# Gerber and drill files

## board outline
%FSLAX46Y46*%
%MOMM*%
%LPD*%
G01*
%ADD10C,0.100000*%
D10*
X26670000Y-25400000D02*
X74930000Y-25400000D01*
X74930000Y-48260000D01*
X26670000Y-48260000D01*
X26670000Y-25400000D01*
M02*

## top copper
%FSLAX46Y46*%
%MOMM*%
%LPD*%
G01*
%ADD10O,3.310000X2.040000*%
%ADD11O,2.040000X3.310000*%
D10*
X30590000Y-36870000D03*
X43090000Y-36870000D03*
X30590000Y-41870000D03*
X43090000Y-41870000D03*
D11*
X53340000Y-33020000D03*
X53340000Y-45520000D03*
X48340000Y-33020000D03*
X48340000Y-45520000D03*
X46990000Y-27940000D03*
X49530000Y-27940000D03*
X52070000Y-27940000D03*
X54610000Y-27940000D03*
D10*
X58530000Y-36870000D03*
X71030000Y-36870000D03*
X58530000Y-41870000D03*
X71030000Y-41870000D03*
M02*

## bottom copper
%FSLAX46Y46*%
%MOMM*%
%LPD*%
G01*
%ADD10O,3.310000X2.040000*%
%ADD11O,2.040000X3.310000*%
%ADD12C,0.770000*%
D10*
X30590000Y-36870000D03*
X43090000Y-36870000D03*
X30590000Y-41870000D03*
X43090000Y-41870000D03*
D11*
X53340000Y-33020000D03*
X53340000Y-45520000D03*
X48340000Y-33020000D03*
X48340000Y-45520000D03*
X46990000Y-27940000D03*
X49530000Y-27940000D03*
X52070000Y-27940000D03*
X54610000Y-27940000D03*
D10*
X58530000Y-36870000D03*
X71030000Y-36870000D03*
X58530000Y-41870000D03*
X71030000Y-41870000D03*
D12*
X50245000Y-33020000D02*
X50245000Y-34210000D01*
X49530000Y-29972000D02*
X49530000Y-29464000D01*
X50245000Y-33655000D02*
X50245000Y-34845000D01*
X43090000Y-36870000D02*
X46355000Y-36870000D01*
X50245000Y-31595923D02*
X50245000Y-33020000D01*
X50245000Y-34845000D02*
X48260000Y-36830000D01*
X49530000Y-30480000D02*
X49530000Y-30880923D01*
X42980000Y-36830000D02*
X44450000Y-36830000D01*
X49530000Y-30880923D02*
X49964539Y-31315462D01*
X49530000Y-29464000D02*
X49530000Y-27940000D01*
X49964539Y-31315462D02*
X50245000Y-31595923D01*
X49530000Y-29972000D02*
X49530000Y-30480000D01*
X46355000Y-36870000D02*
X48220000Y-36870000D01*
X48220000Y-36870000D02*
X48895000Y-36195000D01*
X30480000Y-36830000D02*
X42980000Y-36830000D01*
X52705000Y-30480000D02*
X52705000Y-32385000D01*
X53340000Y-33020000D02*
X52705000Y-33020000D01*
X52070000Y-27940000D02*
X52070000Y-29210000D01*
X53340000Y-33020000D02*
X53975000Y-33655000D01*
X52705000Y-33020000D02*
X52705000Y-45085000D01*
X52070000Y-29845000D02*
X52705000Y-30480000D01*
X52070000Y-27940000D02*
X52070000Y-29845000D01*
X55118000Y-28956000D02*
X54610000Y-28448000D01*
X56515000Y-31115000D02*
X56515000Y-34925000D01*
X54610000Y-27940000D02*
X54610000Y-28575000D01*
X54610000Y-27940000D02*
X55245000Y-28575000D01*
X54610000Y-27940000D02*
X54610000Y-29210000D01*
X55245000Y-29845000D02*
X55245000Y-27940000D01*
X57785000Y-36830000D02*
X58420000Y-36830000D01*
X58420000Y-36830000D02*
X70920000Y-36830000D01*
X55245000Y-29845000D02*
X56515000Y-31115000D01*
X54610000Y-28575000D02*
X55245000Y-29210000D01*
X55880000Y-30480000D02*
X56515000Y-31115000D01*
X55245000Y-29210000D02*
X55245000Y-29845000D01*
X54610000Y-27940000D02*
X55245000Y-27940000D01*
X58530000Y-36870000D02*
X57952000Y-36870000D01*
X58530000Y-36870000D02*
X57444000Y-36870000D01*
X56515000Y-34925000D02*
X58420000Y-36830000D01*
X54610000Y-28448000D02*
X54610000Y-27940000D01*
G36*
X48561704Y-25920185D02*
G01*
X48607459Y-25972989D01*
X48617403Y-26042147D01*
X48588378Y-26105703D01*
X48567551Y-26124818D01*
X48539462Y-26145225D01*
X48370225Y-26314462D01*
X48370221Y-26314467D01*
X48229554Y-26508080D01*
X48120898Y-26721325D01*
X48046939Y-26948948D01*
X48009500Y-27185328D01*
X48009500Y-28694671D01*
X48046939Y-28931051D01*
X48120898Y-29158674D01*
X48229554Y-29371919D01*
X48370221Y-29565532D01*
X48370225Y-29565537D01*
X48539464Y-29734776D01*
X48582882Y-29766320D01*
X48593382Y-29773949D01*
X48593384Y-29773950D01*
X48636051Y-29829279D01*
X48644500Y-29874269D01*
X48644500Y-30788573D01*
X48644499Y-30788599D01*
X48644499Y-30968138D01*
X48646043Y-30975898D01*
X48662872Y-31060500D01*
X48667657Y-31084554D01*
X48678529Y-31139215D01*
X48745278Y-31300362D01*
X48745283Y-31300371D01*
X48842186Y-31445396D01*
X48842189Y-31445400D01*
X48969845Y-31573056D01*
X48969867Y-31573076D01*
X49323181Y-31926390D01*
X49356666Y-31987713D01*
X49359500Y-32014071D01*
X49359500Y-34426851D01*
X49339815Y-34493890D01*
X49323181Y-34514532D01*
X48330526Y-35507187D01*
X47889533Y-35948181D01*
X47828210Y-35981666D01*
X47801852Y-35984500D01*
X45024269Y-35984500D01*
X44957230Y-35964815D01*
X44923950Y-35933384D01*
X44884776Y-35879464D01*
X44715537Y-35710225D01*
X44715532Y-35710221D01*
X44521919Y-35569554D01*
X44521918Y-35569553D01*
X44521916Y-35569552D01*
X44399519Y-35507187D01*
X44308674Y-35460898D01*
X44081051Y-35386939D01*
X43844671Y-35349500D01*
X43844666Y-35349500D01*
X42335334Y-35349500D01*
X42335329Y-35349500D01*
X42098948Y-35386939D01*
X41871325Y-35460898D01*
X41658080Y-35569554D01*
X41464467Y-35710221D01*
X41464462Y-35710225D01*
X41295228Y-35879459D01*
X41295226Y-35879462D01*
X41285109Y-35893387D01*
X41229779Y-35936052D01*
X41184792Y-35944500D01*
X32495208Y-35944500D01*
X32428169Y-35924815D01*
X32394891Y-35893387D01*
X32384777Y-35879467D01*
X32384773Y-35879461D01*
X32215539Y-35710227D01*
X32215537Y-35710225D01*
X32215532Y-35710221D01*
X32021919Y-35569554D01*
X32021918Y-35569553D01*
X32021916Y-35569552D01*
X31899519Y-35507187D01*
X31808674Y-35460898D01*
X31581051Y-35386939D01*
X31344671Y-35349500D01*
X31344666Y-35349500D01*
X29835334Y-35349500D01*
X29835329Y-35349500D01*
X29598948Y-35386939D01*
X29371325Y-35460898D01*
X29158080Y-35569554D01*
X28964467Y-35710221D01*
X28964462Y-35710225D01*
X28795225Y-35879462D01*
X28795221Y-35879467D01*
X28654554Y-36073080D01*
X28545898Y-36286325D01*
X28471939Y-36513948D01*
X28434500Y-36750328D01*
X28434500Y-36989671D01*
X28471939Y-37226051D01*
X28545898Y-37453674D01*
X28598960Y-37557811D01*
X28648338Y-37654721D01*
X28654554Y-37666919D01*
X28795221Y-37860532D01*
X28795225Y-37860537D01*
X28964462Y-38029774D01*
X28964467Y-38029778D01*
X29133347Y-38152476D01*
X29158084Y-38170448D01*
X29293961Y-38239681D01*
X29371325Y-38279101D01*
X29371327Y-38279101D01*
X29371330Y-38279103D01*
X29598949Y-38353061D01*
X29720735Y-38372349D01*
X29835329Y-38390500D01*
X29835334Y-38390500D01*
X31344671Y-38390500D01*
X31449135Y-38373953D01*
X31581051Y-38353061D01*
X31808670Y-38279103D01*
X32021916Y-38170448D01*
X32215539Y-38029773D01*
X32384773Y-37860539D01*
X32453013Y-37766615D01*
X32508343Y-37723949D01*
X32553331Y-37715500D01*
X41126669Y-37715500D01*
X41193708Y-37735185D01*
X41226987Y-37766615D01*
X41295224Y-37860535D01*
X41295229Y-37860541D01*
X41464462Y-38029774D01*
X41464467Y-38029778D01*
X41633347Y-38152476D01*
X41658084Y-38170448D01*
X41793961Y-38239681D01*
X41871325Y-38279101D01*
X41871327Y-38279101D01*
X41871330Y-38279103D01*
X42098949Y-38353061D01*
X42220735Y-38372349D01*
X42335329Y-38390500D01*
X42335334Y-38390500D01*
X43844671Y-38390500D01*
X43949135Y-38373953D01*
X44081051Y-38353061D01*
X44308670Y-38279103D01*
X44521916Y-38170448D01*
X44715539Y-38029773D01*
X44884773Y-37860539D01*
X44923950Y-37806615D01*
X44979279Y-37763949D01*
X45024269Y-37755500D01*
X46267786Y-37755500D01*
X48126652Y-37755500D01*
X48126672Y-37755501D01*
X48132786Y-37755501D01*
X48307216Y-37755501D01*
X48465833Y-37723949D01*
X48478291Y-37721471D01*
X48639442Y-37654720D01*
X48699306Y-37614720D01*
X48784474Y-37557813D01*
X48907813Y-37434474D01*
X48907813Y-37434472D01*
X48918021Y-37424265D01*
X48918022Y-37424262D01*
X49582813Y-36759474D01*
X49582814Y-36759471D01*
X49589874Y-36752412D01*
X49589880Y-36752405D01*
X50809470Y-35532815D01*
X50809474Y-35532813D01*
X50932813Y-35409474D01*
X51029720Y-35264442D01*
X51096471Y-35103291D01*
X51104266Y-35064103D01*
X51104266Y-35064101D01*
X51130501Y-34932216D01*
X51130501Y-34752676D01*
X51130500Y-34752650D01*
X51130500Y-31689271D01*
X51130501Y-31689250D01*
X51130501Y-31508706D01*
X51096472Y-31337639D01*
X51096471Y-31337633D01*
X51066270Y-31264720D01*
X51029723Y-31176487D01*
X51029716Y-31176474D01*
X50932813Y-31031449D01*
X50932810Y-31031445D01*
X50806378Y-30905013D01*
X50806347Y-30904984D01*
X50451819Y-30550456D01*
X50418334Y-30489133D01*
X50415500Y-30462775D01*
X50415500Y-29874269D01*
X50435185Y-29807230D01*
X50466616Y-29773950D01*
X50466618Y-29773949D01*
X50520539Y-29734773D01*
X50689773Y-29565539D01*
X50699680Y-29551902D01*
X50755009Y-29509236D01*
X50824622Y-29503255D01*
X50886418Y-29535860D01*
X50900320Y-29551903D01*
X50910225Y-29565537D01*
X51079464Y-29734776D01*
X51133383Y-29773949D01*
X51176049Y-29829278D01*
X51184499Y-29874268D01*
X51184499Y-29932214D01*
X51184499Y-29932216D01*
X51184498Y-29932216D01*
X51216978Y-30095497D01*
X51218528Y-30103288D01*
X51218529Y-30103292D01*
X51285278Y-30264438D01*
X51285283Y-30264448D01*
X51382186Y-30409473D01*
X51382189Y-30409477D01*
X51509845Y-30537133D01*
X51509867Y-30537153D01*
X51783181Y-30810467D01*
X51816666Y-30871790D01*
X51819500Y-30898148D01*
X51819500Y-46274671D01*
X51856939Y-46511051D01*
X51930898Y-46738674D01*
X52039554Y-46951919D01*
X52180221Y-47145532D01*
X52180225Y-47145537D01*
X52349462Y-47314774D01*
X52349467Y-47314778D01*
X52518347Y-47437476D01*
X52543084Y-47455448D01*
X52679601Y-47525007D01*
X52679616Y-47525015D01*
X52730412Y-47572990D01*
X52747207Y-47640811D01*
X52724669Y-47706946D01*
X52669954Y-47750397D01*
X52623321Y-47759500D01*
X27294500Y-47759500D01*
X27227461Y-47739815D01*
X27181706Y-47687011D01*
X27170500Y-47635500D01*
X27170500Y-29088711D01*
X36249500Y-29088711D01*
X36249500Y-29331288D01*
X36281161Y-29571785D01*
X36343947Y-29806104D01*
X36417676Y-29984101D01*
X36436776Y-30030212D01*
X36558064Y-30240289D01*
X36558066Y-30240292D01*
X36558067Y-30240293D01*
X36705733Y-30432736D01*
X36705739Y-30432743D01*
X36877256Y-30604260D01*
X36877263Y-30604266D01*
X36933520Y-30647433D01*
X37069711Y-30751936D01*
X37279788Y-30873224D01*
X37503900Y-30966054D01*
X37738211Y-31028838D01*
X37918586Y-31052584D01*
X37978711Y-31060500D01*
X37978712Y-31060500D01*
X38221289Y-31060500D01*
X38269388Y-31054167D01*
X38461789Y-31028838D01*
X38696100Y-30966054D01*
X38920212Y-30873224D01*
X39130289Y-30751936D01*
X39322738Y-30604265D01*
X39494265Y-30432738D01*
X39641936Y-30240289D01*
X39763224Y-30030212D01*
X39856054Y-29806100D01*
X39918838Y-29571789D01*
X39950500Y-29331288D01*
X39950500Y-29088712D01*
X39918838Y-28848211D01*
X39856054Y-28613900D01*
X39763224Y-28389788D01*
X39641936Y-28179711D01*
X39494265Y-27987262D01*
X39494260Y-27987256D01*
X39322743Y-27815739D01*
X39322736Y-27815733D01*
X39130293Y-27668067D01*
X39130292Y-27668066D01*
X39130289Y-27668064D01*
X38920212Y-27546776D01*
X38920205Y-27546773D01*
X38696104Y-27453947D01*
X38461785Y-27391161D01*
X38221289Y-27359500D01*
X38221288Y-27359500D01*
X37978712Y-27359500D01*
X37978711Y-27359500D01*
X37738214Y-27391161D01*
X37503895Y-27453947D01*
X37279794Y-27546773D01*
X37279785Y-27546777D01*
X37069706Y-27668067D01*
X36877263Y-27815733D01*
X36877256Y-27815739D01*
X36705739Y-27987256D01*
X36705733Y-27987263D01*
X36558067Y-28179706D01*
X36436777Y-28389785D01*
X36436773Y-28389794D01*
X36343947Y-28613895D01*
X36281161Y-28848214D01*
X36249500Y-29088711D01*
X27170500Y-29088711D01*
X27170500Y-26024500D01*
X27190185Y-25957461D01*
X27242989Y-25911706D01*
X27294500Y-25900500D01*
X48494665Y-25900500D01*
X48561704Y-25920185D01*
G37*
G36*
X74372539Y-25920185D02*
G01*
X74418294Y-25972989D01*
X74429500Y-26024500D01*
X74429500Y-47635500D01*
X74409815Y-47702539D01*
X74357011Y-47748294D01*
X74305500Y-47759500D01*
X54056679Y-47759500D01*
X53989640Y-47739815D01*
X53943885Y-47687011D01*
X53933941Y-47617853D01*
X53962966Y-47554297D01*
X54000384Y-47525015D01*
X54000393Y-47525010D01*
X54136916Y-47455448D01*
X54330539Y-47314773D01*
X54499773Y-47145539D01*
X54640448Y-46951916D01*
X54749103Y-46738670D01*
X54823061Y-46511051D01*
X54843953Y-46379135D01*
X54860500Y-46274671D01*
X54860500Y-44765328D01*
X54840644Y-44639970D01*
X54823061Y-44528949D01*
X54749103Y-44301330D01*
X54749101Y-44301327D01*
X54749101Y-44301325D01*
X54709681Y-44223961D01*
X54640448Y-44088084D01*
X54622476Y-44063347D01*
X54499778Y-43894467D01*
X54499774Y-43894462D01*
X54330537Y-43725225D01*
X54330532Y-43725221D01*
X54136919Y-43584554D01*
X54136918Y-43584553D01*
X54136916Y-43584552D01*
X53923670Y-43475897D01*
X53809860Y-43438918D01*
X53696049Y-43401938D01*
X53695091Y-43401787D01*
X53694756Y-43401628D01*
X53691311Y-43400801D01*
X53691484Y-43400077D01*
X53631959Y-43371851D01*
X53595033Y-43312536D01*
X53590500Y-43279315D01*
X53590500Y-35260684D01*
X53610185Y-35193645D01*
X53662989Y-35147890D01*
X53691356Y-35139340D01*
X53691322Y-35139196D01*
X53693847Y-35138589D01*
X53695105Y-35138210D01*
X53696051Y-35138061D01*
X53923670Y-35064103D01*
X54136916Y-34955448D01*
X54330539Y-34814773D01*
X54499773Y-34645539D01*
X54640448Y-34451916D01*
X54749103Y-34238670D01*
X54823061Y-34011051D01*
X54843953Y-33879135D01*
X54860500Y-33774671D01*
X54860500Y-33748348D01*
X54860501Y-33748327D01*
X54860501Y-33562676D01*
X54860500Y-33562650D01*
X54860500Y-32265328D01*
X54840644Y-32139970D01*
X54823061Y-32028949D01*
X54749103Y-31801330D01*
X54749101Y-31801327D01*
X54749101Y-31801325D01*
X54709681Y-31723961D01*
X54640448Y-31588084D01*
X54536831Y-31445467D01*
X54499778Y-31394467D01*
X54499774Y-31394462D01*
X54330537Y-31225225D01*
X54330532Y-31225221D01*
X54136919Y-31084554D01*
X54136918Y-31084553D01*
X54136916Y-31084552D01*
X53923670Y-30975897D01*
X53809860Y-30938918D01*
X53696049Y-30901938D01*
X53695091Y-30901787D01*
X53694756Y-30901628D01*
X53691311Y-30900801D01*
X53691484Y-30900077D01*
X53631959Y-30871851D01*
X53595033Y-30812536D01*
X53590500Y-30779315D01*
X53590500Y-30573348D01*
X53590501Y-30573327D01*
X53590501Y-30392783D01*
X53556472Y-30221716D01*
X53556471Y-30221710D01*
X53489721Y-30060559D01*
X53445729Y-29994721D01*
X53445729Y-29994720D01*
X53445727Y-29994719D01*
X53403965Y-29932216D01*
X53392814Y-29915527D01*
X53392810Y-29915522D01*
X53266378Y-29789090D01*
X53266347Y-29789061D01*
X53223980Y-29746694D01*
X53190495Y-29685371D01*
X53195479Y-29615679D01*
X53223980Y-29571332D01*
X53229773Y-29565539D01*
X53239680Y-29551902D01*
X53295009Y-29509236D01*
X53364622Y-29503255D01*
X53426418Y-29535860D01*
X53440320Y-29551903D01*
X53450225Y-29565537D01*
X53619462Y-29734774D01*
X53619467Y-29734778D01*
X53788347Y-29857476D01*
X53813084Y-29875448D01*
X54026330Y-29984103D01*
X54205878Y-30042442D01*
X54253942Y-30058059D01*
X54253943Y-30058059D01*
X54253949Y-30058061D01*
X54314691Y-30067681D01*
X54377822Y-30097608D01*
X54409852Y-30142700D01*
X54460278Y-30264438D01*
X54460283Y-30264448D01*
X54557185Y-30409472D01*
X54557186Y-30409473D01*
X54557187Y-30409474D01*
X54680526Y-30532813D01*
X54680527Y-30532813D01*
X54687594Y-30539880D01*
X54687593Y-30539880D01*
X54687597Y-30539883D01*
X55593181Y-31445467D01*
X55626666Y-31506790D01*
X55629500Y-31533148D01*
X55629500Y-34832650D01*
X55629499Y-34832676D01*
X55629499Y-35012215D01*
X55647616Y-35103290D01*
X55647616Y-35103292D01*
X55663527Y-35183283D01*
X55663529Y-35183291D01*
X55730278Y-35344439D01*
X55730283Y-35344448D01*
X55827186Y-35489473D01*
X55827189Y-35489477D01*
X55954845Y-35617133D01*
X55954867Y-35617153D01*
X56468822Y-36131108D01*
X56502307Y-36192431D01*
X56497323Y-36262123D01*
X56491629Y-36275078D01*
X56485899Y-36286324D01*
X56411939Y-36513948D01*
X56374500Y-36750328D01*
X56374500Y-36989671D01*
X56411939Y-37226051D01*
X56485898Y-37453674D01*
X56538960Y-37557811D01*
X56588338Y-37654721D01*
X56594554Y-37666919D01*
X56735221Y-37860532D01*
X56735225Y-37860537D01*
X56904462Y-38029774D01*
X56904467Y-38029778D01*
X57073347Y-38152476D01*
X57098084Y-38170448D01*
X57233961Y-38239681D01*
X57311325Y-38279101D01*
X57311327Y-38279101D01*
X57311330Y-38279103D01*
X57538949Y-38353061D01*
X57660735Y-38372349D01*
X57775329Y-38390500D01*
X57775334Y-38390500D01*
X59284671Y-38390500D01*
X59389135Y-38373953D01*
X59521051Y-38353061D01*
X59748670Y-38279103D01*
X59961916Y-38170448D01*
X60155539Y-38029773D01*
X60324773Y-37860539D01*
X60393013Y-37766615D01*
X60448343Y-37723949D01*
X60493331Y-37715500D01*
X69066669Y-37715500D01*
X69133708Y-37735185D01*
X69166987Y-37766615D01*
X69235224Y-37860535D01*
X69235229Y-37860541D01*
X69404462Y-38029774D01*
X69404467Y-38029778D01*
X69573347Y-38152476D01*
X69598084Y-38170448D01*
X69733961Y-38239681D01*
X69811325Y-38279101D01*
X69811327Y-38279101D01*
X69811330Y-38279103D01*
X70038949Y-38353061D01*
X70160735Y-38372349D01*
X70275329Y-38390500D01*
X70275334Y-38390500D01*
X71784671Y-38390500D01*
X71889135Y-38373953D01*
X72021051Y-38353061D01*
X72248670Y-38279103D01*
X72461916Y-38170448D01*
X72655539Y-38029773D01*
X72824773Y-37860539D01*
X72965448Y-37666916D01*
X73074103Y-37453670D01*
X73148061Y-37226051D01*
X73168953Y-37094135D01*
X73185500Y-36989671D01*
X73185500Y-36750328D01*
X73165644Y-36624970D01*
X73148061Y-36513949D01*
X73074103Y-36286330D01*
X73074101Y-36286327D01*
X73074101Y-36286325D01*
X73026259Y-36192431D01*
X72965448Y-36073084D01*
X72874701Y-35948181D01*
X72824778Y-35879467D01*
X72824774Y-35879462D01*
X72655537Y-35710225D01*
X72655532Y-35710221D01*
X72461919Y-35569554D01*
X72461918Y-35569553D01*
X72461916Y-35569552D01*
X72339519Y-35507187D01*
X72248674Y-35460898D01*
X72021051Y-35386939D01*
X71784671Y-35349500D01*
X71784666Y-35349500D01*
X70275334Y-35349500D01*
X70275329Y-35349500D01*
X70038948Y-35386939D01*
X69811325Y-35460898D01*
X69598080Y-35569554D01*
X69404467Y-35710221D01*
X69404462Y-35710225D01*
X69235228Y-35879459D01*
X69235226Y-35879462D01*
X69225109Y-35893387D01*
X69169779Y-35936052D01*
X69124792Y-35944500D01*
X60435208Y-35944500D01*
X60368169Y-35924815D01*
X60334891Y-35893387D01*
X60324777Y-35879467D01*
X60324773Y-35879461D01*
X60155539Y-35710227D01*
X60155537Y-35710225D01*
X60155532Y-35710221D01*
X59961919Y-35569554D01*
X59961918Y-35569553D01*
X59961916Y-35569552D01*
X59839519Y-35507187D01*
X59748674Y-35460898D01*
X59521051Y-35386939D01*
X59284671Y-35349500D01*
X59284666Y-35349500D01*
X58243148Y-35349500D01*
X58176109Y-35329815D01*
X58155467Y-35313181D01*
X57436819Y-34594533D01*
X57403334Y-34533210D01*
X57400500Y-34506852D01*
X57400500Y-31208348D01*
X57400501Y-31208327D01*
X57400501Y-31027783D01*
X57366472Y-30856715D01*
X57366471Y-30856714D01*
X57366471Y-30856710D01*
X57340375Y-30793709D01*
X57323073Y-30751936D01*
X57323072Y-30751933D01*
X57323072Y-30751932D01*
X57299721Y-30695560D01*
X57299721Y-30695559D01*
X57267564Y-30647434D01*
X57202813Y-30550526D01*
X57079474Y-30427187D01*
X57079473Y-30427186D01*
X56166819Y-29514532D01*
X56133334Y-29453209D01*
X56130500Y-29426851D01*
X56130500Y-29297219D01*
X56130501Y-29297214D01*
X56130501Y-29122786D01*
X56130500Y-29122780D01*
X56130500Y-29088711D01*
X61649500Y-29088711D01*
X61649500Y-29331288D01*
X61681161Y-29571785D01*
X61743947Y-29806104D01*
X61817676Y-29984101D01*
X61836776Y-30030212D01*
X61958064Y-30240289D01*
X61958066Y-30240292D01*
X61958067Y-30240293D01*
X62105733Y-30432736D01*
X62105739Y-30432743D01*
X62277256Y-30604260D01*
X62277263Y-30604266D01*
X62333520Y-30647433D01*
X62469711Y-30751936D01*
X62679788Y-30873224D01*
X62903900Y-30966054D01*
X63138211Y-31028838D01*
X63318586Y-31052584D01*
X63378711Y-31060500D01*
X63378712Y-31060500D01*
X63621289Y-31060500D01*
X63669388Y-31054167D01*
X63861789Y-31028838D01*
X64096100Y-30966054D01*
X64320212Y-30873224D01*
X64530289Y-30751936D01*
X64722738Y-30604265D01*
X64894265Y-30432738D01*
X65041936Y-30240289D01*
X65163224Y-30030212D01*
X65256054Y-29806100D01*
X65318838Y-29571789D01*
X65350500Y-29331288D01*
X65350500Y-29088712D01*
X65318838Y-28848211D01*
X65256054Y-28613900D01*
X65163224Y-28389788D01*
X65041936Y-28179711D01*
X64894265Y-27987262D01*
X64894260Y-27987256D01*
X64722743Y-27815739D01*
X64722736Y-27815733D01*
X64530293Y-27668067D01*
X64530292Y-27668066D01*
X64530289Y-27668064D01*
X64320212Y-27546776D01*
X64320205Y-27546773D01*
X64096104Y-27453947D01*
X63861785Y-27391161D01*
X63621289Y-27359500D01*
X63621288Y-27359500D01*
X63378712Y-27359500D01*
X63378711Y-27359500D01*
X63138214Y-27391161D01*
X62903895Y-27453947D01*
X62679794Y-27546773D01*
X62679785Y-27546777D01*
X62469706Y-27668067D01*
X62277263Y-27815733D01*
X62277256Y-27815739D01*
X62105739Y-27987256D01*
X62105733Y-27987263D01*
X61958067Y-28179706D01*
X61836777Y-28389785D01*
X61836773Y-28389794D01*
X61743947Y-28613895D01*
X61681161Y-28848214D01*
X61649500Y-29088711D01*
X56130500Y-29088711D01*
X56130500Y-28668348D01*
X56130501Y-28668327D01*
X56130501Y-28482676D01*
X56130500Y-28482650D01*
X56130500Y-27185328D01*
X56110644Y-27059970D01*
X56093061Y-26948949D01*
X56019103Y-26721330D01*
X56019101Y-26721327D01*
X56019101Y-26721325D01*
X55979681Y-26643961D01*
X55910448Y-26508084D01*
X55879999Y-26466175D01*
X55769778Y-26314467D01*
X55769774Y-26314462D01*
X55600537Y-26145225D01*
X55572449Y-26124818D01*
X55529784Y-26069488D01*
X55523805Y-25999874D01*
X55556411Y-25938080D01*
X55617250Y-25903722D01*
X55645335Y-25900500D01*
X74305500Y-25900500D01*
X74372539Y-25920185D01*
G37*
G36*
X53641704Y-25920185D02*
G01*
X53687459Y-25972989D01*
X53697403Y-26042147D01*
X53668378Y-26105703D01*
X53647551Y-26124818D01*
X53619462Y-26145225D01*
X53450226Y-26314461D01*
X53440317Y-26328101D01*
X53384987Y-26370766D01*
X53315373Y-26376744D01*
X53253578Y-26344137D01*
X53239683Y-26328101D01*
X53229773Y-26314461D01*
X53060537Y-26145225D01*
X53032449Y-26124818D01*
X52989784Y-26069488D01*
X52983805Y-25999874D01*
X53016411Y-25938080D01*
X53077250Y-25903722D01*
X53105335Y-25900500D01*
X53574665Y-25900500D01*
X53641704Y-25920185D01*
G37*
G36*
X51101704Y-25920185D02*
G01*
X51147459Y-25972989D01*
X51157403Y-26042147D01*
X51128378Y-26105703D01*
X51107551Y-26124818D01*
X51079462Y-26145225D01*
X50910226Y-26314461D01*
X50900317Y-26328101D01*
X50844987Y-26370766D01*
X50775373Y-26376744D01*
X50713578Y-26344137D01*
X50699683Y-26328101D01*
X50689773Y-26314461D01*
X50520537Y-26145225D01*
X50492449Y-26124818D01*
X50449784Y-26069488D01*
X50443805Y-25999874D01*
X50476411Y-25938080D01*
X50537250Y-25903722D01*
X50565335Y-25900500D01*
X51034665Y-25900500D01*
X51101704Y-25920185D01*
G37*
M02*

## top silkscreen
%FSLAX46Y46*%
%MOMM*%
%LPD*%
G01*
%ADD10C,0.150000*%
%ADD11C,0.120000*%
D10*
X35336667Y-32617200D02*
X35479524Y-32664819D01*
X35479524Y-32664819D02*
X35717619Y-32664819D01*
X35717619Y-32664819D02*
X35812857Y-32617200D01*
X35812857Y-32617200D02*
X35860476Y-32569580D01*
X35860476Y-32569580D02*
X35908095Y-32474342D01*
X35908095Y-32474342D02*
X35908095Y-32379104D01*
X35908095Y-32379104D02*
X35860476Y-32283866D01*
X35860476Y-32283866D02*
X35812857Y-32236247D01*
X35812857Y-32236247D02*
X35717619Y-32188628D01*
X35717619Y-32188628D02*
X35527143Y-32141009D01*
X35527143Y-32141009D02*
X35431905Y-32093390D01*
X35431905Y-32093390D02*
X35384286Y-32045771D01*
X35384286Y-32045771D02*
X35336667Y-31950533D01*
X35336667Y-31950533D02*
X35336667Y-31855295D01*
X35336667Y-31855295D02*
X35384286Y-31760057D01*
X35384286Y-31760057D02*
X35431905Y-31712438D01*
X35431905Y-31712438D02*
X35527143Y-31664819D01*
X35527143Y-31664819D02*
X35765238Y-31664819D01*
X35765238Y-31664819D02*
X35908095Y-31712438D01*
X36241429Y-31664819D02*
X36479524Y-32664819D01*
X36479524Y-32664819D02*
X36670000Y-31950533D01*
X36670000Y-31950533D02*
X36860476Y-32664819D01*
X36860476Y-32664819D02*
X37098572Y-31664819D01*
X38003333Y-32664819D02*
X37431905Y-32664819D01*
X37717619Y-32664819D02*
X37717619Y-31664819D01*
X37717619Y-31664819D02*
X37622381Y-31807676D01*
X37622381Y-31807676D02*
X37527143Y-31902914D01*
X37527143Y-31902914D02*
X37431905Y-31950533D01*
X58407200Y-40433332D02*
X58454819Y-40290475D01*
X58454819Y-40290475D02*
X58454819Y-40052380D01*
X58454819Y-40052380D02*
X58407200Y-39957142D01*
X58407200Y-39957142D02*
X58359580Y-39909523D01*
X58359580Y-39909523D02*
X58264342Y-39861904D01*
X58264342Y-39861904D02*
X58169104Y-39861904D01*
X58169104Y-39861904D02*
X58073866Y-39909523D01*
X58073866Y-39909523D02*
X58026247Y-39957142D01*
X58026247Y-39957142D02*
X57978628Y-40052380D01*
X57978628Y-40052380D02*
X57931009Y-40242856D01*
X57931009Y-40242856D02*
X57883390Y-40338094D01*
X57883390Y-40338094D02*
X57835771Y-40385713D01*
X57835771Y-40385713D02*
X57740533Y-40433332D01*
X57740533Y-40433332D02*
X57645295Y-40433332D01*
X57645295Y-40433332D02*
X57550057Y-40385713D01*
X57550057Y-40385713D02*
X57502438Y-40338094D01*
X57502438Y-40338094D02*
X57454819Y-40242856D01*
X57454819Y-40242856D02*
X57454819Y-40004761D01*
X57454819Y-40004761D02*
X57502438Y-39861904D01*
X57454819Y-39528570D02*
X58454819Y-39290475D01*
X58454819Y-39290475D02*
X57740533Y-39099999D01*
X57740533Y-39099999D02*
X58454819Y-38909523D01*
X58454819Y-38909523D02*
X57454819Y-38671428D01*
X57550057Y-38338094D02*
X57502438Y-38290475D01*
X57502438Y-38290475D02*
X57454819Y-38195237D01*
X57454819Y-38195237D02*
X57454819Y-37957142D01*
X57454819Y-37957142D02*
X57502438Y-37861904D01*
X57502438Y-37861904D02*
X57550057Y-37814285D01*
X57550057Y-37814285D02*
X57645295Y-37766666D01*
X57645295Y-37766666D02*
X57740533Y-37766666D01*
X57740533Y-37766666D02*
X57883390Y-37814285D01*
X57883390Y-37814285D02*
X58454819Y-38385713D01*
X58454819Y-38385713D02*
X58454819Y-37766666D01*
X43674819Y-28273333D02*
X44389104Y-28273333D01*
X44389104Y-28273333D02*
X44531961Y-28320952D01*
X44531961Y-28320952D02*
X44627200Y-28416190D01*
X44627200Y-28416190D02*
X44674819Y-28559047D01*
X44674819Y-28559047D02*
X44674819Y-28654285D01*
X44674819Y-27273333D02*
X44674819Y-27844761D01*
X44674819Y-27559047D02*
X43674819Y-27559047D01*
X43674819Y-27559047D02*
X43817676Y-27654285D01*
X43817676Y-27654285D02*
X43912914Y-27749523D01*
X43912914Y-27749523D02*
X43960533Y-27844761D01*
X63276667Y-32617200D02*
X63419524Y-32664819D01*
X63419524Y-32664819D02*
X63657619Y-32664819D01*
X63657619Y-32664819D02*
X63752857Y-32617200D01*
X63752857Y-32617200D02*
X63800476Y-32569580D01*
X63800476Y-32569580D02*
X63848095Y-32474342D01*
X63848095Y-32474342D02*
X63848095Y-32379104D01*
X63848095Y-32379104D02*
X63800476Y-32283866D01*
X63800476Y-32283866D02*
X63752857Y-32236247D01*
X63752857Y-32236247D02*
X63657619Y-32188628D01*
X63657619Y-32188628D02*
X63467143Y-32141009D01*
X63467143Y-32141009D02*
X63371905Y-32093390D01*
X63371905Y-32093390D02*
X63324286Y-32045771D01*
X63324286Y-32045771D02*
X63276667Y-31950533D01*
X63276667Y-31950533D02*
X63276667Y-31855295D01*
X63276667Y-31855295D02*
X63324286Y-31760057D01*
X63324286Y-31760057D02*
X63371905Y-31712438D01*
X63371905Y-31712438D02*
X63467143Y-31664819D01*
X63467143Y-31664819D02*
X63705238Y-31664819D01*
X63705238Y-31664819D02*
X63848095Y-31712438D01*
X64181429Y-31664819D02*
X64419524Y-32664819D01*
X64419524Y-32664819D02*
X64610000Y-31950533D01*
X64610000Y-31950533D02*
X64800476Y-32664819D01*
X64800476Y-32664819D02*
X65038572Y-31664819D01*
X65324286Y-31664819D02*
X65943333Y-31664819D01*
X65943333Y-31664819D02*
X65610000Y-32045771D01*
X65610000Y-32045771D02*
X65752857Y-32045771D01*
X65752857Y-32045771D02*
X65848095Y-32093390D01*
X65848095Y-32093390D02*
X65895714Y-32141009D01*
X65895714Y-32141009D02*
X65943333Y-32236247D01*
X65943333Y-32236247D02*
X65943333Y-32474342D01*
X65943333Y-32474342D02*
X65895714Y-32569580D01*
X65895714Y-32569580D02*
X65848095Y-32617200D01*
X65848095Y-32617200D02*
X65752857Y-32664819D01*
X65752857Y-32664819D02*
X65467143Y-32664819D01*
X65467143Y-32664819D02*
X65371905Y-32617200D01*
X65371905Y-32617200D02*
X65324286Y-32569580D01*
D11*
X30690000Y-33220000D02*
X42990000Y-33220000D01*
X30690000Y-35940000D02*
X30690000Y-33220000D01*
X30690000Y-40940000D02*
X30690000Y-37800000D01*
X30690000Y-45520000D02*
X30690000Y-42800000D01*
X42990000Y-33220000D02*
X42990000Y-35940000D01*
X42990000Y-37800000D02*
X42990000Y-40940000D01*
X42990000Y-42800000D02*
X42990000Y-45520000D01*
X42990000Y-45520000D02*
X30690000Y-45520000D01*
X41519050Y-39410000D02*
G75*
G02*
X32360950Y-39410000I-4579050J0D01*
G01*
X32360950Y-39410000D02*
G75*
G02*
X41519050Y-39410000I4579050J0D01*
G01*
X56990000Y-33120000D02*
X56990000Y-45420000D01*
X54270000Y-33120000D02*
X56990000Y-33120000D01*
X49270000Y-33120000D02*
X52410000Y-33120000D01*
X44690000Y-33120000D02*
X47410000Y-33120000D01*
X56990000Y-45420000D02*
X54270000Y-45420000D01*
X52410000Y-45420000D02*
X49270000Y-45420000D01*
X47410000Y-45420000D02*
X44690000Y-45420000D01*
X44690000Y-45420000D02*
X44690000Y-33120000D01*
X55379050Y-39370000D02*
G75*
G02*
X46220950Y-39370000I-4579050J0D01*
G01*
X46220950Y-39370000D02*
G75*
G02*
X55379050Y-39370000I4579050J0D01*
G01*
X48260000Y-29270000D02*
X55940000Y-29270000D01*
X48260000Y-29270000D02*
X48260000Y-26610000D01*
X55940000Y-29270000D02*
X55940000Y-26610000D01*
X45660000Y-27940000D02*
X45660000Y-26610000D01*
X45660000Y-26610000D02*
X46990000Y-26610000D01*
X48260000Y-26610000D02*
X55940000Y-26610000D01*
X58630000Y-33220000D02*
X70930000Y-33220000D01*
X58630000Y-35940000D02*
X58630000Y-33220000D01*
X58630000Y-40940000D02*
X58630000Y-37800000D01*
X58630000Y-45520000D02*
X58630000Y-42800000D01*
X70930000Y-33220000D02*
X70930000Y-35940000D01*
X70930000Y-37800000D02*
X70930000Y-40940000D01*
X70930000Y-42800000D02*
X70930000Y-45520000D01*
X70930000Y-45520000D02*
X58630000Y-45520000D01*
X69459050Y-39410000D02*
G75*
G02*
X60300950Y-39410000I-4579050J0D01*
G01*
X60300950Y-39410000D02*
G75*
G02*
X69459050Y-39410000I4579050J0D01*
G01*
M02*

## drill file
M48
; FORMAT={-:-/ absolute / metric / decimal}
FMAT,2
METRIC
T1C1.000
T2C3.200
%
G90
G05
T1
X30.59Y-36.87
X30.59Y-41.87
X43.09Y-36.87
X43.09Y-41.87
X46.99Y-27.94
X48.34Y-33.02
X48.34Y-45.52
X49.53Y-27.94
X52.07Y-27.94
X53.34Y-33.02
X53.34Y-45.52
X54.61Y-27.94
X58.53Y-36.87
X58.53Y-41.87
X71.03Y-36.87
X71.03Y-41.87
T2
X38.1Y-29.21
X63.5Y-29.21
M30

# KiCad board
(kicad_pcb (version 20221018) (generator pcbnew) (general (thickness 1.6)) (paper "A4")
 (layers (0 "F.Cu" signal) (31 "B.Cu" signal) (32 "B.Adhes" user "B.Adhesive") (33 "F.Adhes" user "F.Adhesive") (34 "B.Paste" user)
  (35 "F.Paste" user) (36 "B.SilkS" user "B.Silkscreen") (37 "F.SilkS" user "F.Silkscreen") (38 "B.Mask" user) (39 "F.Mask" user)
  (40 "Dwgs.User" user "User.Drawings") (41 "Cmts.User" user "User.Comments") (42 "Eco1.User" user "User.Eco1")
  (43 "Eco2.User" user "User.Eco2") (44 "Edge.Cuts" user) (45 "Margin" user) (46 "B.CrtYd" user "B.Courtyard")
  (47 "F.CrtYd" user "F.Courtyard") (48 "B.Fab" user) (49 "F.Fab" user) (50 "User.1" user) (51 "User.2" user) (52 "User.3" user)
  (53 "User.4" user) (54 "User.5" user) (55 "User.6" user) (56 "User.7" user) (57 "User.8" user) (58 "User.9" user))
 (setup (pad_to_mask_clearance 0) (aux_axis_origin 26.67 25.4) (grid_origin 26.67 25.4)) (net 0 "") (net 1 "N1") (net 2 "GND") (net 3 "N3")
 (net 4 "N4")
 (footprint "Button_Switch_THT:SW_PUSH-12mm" (layer "F.Cu") (at 30.59 36.87)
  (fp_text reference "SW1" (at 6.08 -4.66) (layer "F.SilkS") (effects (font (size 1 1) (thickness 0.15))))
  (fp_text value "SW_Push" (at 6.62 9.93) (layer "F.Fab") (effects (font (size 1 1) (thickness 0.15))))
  (fp_line (start 0.1 -3.65) (end 12.4 -3.65) (stroke (width 0.12) (type solid)) (layer "F.SilkS"))
  (fp_line (start 0.1 -0.93) (end 0.1 -3.65) (stroke (width 0.12) (type solid)) (layer "F.SilkS"))
  (fp_line (start 0.1 4.07) (end 0.1 0.93) (stroke (width 0.12) (type solid)) (layer "F.SilkS"))
  (fp_line (start 0.1 8.65) (end 0.1 5.93) (stroke (width 0.12) (type solid)) (layer "F.SilkS"))
  (fp_line (start 12.4 -3.65) (end 12.4 -0.93) (stroke (width 0.12) (type solid)) (layer "F.SilkS"))
  (fp_line (start 12.4 0.93) (end 12.4 4.07) (stroke (width 0.12) (type solid)) (layer "F.SilkS"))
  (fp_line (start 12.4 5.93) (end 12.4 8.65) (stroke (width 0.12) (type solid)) (layer "F.SilkS"))
  (fp_line (start 12.4 8.65) (end 0.1 8.65) (stroke (width 0.12) (type solid)) (layer "F.SilkS"))
  (fp_circle (center 6.35 2.54) (end 10.16 5.08) (stroke (width 0.12) (type solid)) (fill none) (layer "F.SilkS"))
  (pad "1" thru_hole oval (at 0 0) (size 3.31 2.04) (drill 1) (layers "*.Cu" "*.Mask") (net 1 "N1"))
  (pad "1" thru_hole oval (at 12.5 0) (size 3.31 2.04) (drill 1) (layers "*.Cu" "*.Mask") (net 1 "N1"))
  (pad "2" thru_hole oval (at 0 5) (size 3.31 2.04) (drill 1) (layers "*.Cu" "*.Mask") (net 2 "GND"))
  (pad "2" thru_hole oval (at 12.5 5) (size 3.31 2.04) (drill 1) (layers "*.Cu" "*.Mask") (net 2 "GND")))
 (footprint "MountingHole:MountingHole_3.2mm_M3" (layer "F.Cu") (at 38.1 29.21)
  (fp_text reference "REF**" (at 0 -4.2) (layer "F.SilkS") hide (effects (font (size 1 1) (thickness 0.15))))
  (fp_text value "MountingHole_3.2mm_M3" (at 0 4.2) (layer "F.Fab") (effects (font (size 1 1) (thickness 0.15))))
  (pad "" np_thru_hole circle (at 0 0) (size 3.2 3.2) (drill 3.2) (layers "F&B.Cu" "*.Mask")))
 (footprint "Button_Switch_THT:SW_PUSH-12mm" (layer "F.Cu") (at 53.34 33.02 -90)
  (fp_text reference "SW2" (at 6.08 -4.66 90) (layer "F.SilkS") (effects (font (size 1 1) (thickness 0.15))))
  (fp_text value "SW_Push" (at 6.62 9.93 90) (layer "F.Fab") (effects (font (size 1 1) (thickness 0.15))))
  (fp_line (start 0.1 -3.65) (end 12.4 -3.65) (stroke (width 0.12) (type solid)) (layer "F.SilkS"))
  (fp_line (start 0.1 -0.93) (end 0.1 -3.65) (stroke (width 0.12) (type solid)) (layer "F.SilkS"))
  (fp_line (start 0.1 4.07) (end 0.1 0.93) (stroke (width 0.12) (type solid)) (layer "F.SilkS"))
  (fp_line (start 0.1 8.65) (end 0.1 5.93) (stroke (width 0.12) (type solid)) (layer "F.SilkS"))
  (fp_line (start 12.4 -3.65) (end 12.4 -0.93) (stroke (width 0.12) (type solid)) (layer "F.SilkS"))
  (fp_line (start 12.4 0.93) (end 12.4 4.07) (stroke (width 0.12) (type solid)) (layer "F.SilkS"))
  (fp_line (start 12.4 5.93) (end 12.4 8.65) (stroke (width 0.12) (type solid)) (layer "F.SilkS"))
  (fp_line (start 12.4 8.65) (end 0.1 8.65) (stroke (width 0.12) (type solid)) (layer "F.SilkS"))
  (fp_circle (center 6.35 2.54) (end 10.16 5.08) (stroke (width 0.12) (type solid)) (fill none) (layer "F.SilkS"))
  (pad "1" thru_hole oval (at 0 0 270) (size 3.31 2.04) (drill 1) (layers "*.Cu" "*.Mask") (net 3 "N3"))
  (pad "1" thru_hole oval (at 12.5 0 270) (size 3.31 2.04) (drill 1) (layers "*.Cu" "*.Mask") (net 3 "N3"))
  (pad "2" thru_hole oval (at 0 5 270) (size 3.31 2.04) (drill 1) (layers "*.Cu" "*.Mask") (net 2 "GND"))
  (pad "2" thru_hole oval (at 12.5 5 270) (size 3.31 2.04) (drill 1) (layers "*.Cu" "*.Mask") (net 2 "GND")))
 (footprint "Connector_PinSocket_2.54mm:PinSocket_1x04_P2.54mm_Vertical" (layer "F.Cu") (at 46.99 27.94 90)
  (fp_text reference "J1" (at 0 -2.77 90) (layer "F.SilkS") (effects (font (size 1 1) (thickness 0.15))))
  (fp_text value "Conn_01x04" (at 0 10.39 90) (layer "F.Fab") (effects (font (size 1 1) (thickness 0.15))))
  (fp_line (start -1.33 1.27) (end -1.33 8.95) (stroke (width 0.12) (type solid)) (layer "F.SilkS"))
  (fp_line (start -1.33 1.27) (end 1.33 1.27) (stroke (width 0.12) (type solid)) (layer "F.SilkS"))
  (fp_line (start -1.33 8.95) (end 1.33 8.95) (stroke (width 0.12) (type solid)) (layer "F.SilkS"))
  (fp_line (start 0 -1.33) (end 1.33 -1.33) (stroke (width 0.12) (type solid)) (layer "F.SilkS"))
  (fp_line (start 1.33 -1.33) (end 1.33 0) (stroke (width 0.12) (type solid)) (layer "F.SilkS"))
  (fp_line (start 1.33 1.27) (end 1.33 8.95) (stroke (width 0.12) (type solid)) (layer "F.SilkS"))
  (pad "1" thru_hole oval (at 0 0 90) (size 3.31 2.04) (drill 1) (layers "*.Cu" "*.Mask") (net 2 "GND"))
  (pad "2" thru_hole oval (at 0 2.54 90) (size 3.31 2.04) (drill 1) (layers "*.Cu" "*.Mask") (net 1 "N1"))
  (pad "3" thru_hole oval (at 0 5.08 90) (size 3.31 2.04) (drill 1) (layers "*.Cu" "*.Mask") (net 3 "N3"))
  (pad "4" thru_hole oval (at 0 7.62 90) (size 3.31 2.04) (drill 1) (layers "*.Cu" "*.Mask") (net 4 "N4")))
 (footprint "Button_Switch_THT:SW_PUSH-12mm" (layer "F.Cu") (at 58.53 36.87)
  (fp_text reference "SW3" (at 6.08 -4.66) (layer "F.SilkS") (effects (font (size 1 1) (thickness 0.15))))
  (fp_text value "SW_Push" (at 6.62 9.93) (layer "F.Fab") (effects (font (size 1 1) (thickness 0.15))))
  (fp_line (start 0.1 -3.65) (end 12.4 -3.65) (stroke (width 0.12) (type solid)) (layer "F.SilkS"))
  (fp_line (start 0.1 -0.93) (end 0.1 -3.65) (stroke (width 0.12) (type solid)) (layer "F.SilkS"))
  (fp_line (start 0.1 4.07) (end 0.1 0.93) (stroke (width 0.12) (type solid)) (layer "F.SilkS"))
  (fp_line (start 0.1 8.65) (end 0.1 5.93) (stroke (width 0.12) (type solid)) (layer "F.SilkS"))
  (fp_line (start 12.4 -3.65) (end 12.4 -0.93) (stroke (width 0.12) (type solid)) (layer "F.SilkS"))
  (fp_line (start 12.4 0.93) (end 12.4 4.07) (stroke (width 0.12) (type solid)) (layer "F.SilkS"))
  (fp_line (start 12.4 5.93) (end 12.4 8.65) (stroke (width 0.12) (type solid)) (layer "F.SilkS"))
  (fp_line (start 12.4 8.65) (end 0.1 8.65) (stroke (width 0.12) (type solid)) (layer "F.SilkS"))
  (fp_circle (center 6.35 2.54) (end 10.16 5.08) (stroke (width 0.12) (type solid)) (fill none) (layer "F.SilkS"))
  (pad "1" thru_hole oval (at 0 0) (size 3.31 2.04) (drill 1) (layers "*.Cu" "*.Mask") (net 4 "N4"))
  (pad "1" thru_hole oval (at 12.5 0) (size 3.31 2.04) (drill 1) (layers "*.Cu" "*.Mask") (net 4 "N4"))
  (pad "2" thru_hole oval (at 0 5) (size 3.31 2.04) (drill 1) (layers "*.Cu" "*.Mask") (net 2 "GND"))
  (pad "2" thru_hole oval (at 12.5 5) (size 3.31 2.04) (drill 1) (layers "*.Cu" "*.Mask") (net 2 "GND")))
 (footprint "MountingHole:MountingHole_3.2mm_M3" (layer "F.Cu") (at 63.5 29.21)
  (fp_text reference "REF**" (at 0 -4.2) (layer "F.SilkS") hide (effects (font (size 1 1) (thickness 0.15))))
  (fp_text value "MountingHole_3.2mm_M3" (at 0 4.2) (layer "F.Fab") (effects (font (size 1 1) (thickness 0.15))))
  (pad "" np_thru_hole circle (at 0 0) (size 3.2 3.2) (drill 3.2) (layers "F&B.Cu" "*.Mask")))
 (gr_rect (start 26.67 25.4) (end 74.93 48.26) (stroke (width 0.1) (type default)) (fill none) (layer "Edge.Cuts"))
 (segment (start 50.245 33.02) (end 50.245 34.21) (width 0.77) (layer "B.Cu") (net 1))
 (segment (start 49.53 29.972) (end 49.53 29.464) (width 0.77) (layer "B.Cu") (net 1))
 (segment (start 50.245 33.655) (end 50.245 34.845) (width 0.77) (layer "B.Cu") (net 1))
 (segment (start 43.09 36.87) (end 46.355 36.87) (width 0.77) (layer "B.Cu") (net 1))
 (segment (start 50.245 31.595923) (end 50.245 33.02) (width 0.77) (layer "B.Cu") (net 1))
 (segment (start 50.245 34.845) (end 48.26 36.83) (width 0.77) (layer "B.Cu") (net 1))
 (segment (start 49.53 30.48) (end 49.53 30.880923) (width 0.77) (layer "B.Cu") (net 1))
 (segment (start 42.98 36.83) (end 44.45 36.83) (width 0.77) (layer "B.Cu") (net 1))
 (segment (start 49.53 30.880923) (end 49.964539 31.315462) (width 0.77) (layer "B.Cu") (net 1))
 (segment (start 49.53 29.464) (end 49.53 27.94) (width 0.77) (layer "B.Cu") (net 1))
 (segment (start 49.964539 31.315462) (end 50.245 31.595923) (width 0.77) (layer "B.Cu") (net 1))
 (segment (start 49.53 29.972) (end 49.53 30.48) (width 0.77) (layer "B.Cu") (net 1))
 (segment (start 46.355 36.87) (end 48.22 36.87) (width 0.77) (layer "B.Cu") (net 1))
 (segment (start 48.22 36.87) (end 48.895 36.195) (width 0.77) (layer "B.Cu") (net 1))
 (segment (start 30.48 36.83) (end 42.98 36.83) (width 0.77) (layer "B.Cu") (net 1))
 (segment (start 52.705 30.48) (end 52.705 32.385) (width 0.77) (layer "B.Cu") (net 3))
 (segment (start 53.34 33.02) (end 52.705 33.02) (width 0.77) (layer "B.Cu") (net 3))
 (segment (start 52.07 27.94) (end 52.07 29.21) (width 0.77) (layer "B.Cu") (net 3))
 (segment (start 53.34 33.02) (end 53.975 33.655) (width 0.77) (layer "B.Cu") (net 3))
 (segment (start 52.705 33.02) (end 52.705 45.085) (width 0.77) (layer "B.Cu") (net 3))
 (segment (start 52.07 29.845) (end 52.705 30.48) (width 0.77) (layer "B.Cu") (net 3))
 (segment (start 52.07 27.94) (end 52.07 29.845) (width 0.77) (layer "B.Cu") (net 3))
 (segment (start 55.118 28.956) (end 54.61 28.448) (width 0.77) (layer "B.Cu") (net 4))
 (segment (start 56.515 31.115) (end 56.515 34.925) (width 0.77) (layer "B.Cu") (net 4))
 (segment (start 54.61 27.94) (end 54.61 28.575) (width 0.77) (layer "B.Cu") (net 4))
 (segment (start 54.61 27.94) (end 55.245 28.575) (width 0.77) (layer "B.Cu") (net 4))
 (segment (start 54.61 27.94) (end 54.61 29.21) (width 0.77) (layer "B.Cu") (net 4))
 (segment (start 55.245 29.845) (end 55.245 27.94) (width 0.77) (layer "B.Cu") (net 4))
 (segment (start 57.785 36.83) (end 58.42 36.83) (width 0.77) (layer "B.Cu") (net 4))
 (segment (start 58.42 36.83) (end 70.92 36.83) (width 0.77) (layer "B.Cu") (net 4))
 (segment (start 55.245 29.845) (end 56.515 31.115) (width 0.77) (layer "B.Cu") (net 4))
 (segment (start 54.61 28.575) (end 55.245 29.21) (width 0.77) (layer "B.Cu") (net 4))
 (segment (start 55.88 30.48) (end 56.515 31.115) (width 0.77) (layer "B.Cu") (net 4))
 (segment (start 55.245 29.21) (end 55.245 29.845) (width 0.77) (layer "B.Cu") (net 4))
 (segment (start 54.61 27.94) (end 55.245 27.94) (width 0.77) (layer "B.Cu") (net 4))
 (segment (start 58.53 36.87) (end 57.952 36.87) (width 0.77) (layer "B.Cu") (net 4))
 (segment (start 58.53 36.87) (end 57.444 36.87) (width 0.77) (layer "B.Cu") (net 4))
 (segment (start 56.515 34.925) (end 58.42 36.83) (width 0.77) (layer "B.Cu") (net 4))
 (segment (start 54.61 28.448) (end 54.61 27.94) (width 0.77) (layer "B.Cu") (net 4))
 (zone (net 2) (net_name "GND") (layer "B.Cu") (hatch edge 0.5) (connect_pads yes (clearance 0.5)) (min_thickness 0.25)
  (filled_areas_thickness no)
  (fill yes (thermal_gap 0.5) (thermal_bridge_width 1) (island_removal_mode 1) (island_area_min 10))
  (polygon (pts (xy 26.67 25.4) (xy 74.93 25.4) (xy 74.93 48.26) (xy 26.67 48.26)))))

